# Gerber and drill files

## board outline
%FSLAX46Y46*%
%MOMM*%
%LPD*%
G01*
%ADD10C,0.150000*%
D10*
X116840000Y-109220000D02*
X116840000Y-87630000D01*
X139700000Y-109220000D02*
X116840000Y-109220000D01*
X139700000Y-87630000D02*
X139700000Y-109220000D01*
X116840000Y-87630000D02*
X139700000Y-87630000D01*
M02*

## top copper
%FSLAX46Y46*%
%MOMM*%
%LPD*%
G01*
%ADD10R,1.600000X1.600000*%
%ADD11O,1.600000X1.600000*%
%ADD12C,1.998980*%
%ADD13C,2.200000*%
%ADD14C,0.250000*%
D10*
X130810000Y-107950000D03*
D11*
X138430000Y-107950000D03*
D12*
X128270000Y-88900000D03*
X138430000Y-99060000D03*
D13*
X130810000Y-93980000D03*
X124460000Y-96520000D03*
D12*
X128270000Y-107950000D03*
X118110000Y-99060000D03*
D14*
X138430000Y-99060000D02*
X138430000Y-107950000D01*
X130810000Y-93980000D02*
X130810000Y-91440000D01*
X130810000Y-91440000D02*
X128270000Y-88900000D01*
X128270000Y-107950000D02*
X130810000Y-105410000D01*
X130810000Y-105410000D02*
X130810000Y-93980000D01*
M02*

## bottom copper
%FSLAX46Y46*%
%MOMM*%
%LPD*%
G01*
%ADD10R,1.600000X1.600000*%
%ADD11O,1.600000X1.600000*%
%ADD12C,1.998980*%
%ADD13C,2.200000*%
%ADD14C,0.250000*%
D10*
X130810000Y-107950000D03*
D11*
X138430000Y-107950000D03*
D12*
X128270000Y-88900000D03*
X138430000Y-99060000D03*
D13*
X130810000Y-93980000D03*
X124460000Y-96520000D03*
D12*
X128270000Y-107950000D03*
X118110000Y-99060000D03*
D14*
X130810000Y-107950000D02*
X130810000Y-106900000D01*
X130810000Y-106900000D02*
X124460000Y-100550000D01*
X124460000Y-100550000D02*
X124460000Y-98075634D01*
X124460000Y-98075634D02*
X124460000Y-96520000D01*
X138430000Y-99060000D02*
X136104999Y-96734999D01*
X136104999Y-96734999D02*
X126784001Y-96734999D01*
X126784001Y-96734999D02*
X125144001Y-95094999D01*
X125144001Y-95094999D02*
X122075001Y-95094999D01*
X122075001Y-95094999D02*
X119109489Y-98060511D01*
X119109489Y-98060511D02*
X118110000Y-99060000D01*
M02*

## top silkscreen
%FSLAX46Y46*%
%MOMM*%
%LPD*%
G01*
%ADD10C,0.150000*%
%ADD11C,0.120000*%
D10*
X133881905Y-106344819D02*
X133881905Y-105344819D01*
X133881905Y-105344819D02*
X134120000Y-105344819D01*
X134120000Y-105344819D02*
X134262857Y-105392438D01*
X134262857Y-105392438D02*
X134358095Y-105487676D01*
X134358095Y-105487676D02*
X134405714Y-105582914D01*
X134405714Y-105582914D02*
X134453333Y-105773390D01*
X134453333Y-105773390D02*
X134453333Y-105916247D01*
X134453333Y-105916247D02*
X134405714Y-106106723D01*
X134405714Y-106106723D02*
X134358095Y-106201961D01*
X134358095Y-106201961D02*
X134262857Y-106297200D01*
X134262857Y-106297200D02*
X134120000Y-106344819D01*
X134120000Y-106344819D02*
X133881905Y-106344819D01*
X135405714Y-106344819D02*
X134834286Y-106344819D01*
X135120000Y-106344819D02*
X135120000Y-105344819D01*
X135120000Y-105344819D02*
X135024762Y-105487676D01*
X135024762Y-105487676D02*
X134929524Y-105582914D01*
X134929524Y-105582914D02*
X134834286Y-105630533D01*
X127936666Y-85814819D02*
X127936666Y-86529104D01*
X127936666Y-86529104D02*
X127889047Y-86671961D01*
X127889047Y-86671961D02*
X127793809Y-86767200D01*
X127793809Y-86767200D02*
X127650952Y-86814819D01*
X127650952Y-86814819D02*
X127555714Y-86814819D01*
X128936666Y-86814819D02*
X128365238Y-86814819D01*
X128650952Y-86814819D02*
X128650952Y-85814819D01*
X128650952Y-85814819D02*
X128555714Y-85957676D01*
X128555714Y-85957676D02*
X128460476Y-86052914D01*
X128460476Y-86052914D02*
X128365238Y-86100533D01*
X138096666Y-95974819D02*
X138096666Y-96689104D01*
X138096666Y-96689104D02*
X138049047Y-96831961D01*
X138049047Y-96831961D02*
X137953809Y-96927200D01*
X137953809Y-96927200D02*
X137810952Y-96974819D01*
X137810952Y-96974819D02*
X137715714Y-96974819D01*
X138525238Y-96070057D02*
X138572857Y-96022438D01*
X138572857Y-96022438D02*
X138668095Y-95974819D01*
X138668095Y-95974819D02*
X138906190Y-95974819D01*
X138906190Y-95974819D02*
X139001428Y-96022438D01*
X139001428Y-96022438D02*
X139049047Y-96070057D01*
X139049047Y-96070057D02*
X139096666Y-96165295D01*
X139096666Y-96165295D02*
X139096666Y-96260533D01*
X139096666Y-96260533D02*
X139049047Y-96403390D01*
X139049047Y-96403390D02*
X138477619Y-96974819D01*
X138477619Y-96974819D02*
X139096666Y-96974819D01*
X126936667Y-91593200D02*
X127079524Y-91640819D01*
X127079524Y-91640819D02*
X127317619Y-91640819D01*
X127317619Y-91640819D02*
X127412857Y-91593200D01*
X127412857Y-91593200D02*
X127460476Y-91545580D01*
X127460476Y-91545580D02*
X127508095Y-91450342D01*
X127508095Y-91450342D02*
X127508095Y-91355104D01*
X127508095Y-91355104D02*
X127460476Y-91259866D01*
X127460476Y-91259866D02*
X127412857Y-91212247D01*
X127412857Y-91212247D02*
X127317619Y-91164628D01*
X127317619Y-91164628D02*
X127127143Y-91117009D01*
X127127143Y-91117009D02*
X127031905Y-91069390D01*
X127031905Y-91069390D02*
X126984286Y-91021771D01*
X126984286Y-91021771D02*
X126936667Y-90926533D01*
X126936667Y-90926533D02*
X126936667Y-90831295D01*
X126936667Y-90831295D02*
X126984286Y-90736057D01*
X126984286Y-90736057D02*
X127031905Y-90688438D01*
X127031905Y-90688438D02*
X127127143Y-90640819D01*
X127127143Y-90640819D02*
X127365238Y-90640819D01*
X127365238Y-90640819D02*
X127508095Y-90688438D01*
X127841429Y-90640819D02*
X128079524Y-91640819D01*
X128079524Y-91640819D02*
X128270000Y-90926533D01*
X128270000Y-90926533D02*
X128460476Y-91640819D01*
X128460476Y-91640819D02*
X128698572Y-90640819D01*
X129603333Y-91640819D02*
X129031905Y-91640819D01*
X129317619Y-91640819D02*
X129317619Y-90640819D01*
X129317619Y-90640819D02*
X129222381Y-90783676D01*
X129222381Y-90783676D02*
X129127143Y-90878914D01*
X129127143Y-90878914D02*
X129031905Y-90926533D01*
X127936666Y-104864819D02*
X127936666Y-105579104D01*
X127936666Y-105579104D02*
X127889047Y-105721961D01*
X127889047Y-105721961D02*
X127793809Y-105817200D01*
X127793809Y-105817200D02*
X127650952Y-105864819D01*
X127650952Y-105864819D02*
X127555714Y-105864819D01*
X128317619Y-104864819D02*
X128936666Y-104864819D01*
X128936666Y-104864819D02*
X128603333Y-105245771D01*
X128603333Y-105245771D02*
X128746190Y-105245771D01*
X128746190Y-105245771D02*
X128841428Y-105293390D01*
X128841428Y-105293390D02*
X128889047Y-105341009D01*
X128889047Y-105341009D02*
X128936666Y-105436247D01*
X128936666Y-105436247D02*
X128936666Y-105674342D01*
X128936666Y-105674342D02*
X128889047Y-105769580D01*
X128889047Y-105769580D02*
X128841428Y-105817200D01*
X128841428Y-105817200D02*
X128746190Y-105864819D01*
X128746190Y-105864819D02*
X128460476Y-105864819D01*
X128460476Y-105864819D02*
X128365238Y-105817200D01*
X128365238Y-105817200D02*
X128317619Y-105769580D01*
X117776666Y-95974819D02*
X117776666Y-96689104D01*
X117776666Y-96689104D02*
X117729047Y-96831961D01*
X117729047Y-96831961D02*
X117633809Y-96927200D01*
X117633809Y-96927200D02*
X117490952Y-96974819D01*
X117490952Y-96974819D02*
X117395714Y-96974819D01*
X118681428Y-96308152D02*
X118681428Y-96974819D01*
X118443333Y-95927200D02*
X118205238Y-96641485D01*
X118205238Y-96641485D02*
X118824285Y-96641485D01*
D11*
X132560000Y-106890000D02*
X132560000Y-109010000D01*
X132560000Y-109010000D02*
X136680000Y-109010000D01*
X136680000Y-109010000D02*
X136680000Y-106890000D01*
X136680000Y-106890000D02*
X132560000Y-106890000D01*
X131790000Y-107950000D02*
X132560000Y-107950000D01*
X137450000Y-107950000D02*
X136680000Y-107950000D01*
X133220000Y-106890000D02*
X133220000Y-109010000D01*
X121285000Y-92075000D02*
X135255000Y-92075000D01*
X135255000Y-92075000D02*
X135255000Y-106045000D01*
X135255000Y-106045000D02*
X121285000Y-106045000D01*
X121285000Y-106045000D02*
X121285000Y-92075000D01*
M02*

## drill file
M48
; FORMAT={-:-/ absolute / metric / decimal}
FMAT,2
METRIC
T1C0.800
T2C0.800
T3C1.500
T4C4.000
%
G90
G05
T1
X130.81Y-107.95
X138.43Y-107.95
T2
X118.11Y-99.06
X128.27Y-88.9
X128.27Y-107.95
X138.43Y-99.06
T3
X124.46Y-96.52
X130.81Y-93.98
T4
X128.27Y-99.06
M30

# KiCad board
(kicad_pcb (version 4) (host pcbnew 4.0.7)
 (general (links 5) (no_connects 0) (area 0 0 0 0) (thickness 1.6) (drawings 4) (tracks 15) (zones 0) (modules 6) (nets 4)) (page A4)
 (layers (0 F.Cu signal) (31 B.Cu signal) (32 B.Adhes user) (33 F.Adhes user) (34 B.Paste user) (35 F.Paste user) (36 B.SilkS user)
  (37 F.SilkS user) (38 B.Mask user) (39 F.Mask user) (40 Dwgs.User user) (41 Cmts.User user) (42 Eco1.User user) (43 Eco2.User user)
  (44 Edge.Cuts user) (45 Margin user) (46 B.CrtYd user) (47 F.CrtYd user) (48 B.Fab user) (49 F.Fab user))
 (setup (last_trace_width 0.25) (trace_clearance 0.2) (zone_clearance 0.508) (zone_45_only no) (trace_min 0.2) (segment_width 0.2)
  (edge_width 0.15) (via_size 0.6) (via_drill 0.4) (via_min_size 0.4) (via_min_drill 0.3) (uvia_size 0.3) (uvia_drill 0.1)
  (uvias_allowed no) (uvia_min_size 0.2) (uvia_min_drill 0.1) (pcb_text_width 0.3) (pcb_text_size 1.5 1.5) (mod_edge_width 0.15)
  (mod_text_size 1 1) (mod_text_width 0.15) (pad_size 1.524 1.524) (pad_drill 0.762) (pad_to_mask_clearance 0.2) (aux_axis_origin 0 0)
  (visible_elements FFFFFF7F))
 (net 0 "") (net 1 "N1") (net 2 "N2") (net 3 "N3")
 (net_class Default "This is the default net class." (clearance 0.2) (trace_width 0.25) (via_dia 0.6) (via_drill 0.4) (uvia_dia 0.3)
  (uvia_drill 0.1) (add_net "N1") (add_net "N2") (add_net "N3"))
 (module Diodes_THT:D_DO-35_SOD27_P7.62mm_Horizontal (layer F.Cu) (at 130.81 107.95)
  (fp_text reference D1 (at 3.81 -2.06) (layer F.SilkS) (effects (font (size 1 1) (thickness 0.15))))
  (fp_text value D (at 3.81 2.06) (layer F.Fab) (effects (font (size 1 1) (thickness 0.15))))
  (fp_line (start 1.75 -1.06) (end 1.75 1.06) (layer F.SilkS) (width 0.12))
  (fp_line (start 1.75 1.06) (end 5.87 1.06) (layer F.SilkS) (width 0.12))
  (fp_line (start 5.87 1.06) (end 5.87 -1.06) (layer F.SilkS) (width 0.12))
  (fp_line (start 5.87 -1.06) (end 1.75 -1.06) (layer F.SilkS) (width 0.12))
  (fp_line (start 0.98 0) (end 1.75 0) (layer F.SilkS) (width 0.12))
  (fp_line (start 6.64 0) (end 5.87 0) (layer F.SilkS) (width 0.12))
  (fp_line (start 2.41 -1.06) (end 2.41 1.06) (layer F.SilkS) (width 0.12))
  (pad 1 thru_hole rect (at 0 0) (size 1.6 1.6) (drill 0.8) (layers *.Cu *.Mask) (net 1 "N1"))
  (pad 2 thru_hole oval (at 7.62 0) (size 1.6 1.6) (drill 0.8) (layers *.Cu *.Mask) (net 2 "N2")))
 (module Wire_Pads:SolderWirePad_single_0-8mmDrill (layer F.Cu) (at 128.27 88.9)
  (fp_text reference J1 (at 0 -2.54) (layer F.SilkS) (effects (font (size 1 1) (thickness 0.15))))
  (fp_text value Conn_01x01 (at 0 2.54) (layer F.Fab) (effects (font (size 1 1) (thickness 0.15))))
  (pad 1 thru_hole circle (at 0 0) (size 1.99898 1.99898) (drill 0.8001) (layers *.Cu *.Mask) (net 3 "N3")))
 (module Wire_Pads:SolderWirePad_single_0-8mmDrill (layer F.Cu) (at 138.43 99.06)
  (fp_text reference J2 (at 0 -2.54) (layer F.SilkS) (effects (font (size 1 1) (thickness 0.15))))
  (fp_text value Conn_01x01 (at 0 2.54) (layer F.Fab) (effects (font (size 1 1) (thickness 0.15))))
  (pad 1 thru_hole circle (at 0 0) (size 1.99898 1.99898) (drill 0.8001) (layers *.Cu *.Mask) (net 2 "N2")))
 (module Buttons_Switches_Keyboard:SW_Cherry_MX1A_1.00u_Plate (layer F.Cu) (at 130.81 93.98)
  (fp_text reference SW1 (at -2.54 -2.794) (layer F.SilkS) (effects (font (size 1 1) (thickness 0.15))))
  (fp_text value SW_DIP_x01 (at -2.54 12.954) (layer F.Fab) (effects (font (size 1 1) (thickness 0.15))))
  (fp_line (start -9.525 -1.905) (end 4.445 -1.905) (layer F.SilkS) (width 0.12))
  (fp_line (start 4.445 -1.905) (end 4.445 12.065) (layer F.SilkS) (width 0.12))
  (fp_line (start 4.445 12.065) (end -9.525 12.065) (layer F.SilkS) (width 0.12))
  (fp_line (start -9.525 12.065) (end -9.525 -1.905) (layer F.SilkS) (width 0.12))
  (pad 1 thru_hole circle (at 0 0) (size 2.2 2.2) (drill 1.5) (layers *.Cu *.Mask) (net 3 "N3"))
  (pad 2 thru_hole circle (at -6.35 2.54) (size 2.2 2.2) (drill 1.5) (layers *.Cu *.Mask) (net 1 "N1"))
  (pad "" np_thru_hole circle (at -2.54 5.08) (size 4 4) (drill 4) (layers *.Cu *.Mask)))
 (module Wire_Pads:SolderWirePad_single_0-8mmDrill (layer F.Cu) (at 128.27 107.95)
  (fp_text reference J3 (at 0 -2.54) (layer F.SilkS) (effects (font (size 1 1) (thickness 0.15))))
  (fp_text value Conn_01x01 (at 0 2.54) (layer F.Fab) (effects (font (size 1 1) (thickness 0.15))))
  (pad 1 thru_hole circle (at 0 0) (size 1.99898 1.99898) (drill 0.8001) (layers *.Cu *.Mask) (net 3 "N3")))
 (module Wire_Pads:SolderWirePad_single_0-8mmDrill (layer F.Cu) (at 118.11 99.06)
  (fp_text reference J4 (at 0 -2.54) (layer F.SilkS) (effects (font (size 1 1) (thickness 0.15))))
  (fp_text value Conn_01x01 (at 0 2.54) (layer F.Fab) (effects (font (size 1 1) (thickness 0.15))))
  (pad 1 thru_hole circle (at 0 0) (size 1.99898 1.99898) (drill 0.8001) (layers *.Cu *.Mask) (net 2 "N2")))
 (gr_line (start 116.84 109.22) (end 116.84 87.63) (layer Edge.Cuts) (width 0.15))
 (gr_line (start 139.7 109.22) (end 116.84 109.22) (layer Edge.Cuts) (width 0.15))
 (gr_line (start 139.7 87.63) (end 139.7 109.22) (layer Edge.Cuts) (width 0.15))
 (gr_line (start 116.84 87.63) (end 139.7 87.63) (layer Edge.Cuts) (width 0.15))
 (segment (start 130.81 107.95) (end 130.81 106.9) (width 0.25) (layer B.Cu) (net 1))
 (segment (start 130.81 106.9) (end 124.46 100.55) (width 0.25) (layer B.Cu) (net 1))
 (segment (start 124.46 100.55) (end 124.46 98.075634) (width 0.25) (layer B.Cu) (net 1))
 (segment (start 124.46 98.075634) (end 124.46 96.52) (width 0.25) (layer B.Cu) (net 1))
 (segment (start 138.43 99.06) (end 136.104999 96.734999) (width 0.25) (layer B.Cu) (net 2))
 (segment (start 136.104999 96.734999) (end 126.784001 96.734999) (width 0.25) (layer B.Cu) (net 2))
 (segment (start 126.784001 96.734999) (end 125.144001 95.094999) (width 0.25) (layer B.Cu) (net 2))
 (segment (start 125.144001 95.094999) (end 122.075001 95.094999) (width 0.25) (layer B.Cu) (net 2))
 (segment (start 122.075001 95.094999) (end 119.109489 98.060511) (width 0.25) (layer B.Cu) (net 2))
 (segment (start 119.109489 98.060511) (end 118.11 99.06) (width 0.25) (layer B.Cu) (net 2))
 (segment (start 138.43 99.06) (end 138.43 107.95) (width 0.25) (layer F.Cu) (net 2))
 (segment (start 130.81 93.98) (end 130.81 91.44) (width 0.25) (layer F.Cu) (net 3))
 (segment (start 130.81 91.44) (end 128.27 88.9) (width 0.25) (layer F.Cu) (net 3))
 (segment (start 128.27 107.95) (end 130.81 105.41) (width 0.25) (layer F.Cu) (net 3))
 (segment (start 130.81 105.41) (end 130.81 93.98) (width 0.25) (layer F.Cu) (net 3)))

